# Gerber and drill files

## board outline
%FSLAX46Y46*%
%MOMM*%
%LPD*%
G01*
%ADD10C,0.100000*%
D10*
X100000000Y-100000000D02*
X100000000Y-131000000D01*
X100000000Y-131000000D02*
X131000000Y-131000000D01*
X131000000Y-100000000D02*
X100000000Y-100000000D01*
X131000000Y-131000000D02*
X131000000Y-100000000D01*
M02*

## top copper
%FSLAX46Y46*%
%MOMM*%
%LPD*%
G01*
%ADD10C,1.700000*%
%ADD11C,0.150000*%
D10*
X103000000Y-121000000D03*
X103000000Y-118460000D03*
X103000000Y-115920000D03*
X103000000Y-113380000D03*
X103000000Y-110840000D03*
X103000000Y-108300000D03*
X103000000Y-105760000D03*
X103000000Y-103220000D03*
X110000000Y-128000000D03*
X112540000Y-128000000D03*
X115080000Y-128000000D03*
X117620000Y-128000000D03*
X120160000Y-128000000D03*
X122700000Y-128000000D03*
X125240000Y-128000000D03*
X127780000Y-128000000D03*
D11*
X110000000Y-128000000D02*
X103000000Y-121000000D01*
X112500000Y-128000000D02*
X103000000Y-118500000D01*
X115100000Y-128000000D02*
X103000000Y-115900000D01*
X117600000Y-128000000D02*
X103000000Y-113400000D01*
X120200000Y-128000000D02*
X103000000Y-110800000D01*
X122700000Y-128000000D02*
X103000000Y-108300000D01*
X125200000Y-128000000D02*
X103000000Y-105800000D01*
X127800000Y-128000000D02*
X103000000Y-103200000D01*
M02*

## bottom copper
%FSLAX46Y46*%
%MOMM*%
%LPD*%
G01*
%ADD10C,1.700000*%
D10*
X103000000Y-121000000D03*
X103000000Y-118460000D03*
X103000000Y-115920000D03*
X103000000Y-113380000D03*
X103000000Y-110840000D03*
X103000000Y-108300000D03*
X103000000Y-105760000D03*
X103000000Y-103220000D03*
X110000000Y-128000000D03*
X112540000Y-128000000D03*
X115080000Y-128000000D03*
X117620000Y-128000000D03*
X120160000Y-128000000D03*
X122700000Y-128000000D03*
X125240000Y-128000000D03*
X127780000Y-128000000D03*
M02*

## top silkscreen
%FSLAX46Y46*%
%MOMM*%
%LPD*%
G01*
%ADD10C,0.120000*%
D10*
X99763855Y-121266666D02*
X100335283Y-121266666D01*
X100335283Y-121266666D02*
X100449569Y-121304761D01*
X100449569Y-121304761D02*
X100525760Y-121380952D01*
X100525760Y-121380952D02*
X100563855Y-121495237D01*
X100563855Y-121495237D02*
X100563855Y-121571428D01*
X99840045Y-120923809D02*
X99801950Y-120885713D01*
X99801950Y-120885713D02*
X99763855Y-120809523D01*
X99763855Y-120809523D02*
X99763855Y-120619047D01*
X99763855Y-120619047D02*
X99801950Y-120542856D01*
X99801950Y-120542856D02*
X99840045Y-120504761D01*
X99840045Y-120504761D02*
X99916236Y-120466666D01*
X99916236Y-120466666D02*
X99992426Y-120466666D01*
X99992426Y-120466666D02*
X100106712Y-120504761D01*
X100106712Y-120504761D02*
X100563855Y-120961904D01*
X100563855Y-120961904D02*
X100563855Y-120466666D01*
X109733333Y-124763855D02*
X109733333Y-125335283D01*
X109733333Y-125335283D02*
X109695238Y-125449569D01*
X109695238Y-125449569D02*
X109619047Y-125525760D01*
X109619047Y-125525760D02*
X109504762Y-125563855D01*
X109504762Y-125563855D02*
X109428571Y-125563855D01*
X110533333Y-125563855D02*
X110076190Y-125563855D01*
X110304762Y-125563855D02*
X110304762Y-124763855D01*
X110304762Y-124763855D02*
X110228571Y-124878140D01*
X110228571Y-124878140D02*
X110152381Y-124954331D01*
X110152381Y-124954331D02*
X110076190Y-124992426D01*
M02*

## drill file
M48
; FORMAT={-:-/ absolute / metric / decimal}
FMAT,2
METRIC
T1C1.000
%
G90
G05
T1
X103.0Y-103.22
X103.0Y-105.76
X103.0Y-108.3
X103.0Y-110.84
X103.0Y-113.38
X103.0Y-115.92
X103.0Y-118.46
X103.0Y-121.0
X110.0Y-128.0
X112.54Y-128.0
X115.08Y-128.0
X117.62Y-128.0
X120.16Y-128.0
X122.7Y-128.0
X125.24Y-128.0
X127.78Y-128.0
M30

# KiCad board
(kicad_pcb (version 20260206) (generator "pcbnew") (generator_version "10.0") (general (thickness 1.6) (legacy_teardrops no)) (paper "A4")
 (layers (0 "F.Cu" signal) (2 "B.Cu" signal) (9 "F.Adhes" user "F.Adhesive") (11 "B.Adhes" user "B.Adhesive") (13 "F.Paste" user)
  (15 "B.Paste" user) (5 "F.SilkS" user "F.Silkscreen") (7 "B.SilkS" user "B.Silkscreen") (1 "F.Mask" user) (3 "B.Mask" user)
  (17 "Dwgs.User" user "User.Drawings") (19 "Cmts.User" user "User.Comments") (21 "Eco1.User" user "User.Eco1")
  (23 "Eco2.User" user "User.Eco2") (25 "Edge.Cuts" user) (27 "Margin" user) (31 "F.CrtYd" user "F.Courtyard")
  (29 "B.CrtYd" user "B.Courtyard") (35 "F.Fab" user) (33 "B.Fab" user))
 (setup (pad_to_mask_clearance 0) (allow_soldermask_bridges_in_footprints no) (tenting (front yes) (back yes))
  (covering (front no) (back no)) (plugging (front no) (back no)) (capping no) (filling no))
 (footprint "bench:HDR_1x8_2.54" (layer "F.Cu") (at 103 121 90)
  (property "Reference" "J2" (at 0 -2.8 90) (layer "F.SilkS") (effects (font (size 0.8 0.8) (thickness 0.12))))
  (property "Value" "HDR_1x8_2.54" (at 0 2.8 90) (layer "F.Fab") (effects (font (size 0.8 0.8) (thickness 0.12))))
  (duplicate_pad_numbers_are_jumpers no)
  (pad "1" thru_hole circle (at 0 0 90) (size 1.7 1.7) (drill 1) (layers "*.Cu" "*.Mask") (remove_unused_layers no) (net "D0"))
  (pad "2" thru_hole circle (at 2.54 0 90) (size 1.7 1.7) (drill 1) (layers "*.Cu" "*.Mask") (remove_unused_layers no) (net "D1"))
  (pad "3" thru_hole circle (at 5.08 0 90) (size 1.7 1.7) (drill 1) (layers "*.Cu" "*.Mask") (remove_unused_layers no) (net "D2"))
  (pad "4" thru_hole circle (at 7.62 0 90) (size 1.7 1.7) (drill 1) (layers "*.Cu" "*.Mask") (remove_unused_layers no) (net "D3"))
  (pad "5" thru_hole circle (at 10.16 0 90) (size 1.7 1.7) (drill 1) (layers "*.Cu" "*.Mask") (remove_unused_layers no) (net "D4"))
  (pad "6" thru_hole circle (at 12.7 0 90) (size 1.7 1.7) (drill 1) (layers "*.Cu" "*.Mask") (remove_unused_layers no) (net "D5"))
  (pad "7" thru_hole circle (at 15.24 0 90) (size 1.7 1.7) (drill 1) (layers "*.Cu" "*.Mask") (remove_unused_layers no) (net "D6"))
  (pad "8" thru_hole circle (at 17.78 0 90) (size 1.7 1.7) (drill 1) (layers "*.Cu" "*.Mask") (remove_unused_layers no) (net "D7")))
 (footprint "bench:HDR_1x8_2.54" (layer "F.Cu") (at 110 128)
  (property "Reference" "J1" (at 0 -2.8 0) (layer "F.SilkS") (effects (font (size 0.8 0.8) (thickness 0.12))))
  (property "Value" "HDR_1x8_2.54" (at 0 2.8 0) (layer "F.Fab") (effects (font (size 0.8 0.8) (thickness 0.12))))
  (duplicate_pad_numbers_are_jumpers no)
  (pad "1" thru_hole circle (at 0 0) (size 1.7 1.7) (drill 1) (layers "*.Cu" "*.Mask") (remove_unused_layers no) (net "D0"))
  (pad "2" thru_hole circle (at 2.54 0) (size 1.7 1.7) (drill 1) (layers "*.Cu" "*.Mask") (remove_unused_layers no) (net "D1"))
  (pad "3" thru_hole circle (at 5.08 0) (size 1.7 1.7) (drill 1) (layers "*.Cu" "*.Mask") (remove_unused_layers no) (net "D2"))
  (pad "4" thru_hole circle (at 7.62 0) (size 1.7 1.7) (drill 1) (layers "*.Cu" "*.Mask") (remove_unused_layers no) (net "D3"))
  (pad "5" thru_hole circle (at 10.16 0) (size 1.7 1.7) (drill 1) (layers "*.Cu" "*.Mask") (remove_unused_layers no) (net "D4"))
  (pad "6" thru_hole circle (at 12.7 0) (size 1.7 1.7) (drill 1) (layers "*.Cu" "*.Mask") (remove_unused_layers no) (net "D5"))
  (pad "7" thru_hole circle (at 15.24 0) (size 1.7 1.7) (drill 1) (layers "*.Cu" "*.Mask") (remove_unused_layers no) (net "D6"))
  (pad "8" thru_hole circle (at 17.78 0) (size 1.7 1.7) (drill 1) (layers "*.Cu" "*.Mask") (remove_unused_layers no) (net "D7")))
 (gr_line (start 100 100) (end 100 131) (stroke (width 0.1) (type solid)) (layer "Edge.Cuts"))
 (gr_line (start 100 131) (end 131 131) (stroke (width 0.1) (type solid)) (layer "Edge.Cuts"))
 (gr_line (start 131 100) (end 100 100) (stroke (width 0.1) (type solid)) (layer "Edge.Cuts"))
 (gr_line (start 131 131) (end 131 100) (stroke (width 0.1) (type solid)) (layer "Edge.Cuts"))
 (segment (start 110 128) (end 103 121) (width 0.15) (layer "F.Cu") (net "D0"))
 (segment (start 112.5 128) (end 103 118.5) (width 0.15) (layer "F.Cu") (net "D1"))
 (segment (start 115.1 128) (end 103 115.9) (width 0.15) (layer "F.Cu") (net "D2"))
 (segment (start 117.6 128) (end 103 113.4) (width 0.15) (layer "F.Cu") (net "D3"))
 (segment (start 120.2 128) (end 103 110.8) (width 0.15) (layer "F.Cu") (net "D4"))
 (segment (start 122.7 128) (end 103 108.3) (width 0.15) (layer "F.Cu") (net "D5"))
 (segment (start 125.2 128) (end 103 105.8) (width 0.15) (layer "F.Cu") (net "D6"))
 (segment (start 127.8 128) (end 103 103.2) (width 0.15) (layer "F.Cu") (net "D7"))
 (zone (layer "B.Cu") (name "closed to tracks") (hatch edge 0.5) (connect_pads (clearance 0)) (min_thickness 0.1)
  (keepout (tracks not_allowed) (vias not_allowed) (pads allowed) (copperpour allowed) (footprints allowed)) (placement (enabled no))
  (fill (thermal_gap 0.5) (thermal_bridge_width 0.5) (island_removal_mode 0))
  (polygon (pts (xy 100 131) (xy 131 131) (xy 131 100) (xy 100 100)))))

